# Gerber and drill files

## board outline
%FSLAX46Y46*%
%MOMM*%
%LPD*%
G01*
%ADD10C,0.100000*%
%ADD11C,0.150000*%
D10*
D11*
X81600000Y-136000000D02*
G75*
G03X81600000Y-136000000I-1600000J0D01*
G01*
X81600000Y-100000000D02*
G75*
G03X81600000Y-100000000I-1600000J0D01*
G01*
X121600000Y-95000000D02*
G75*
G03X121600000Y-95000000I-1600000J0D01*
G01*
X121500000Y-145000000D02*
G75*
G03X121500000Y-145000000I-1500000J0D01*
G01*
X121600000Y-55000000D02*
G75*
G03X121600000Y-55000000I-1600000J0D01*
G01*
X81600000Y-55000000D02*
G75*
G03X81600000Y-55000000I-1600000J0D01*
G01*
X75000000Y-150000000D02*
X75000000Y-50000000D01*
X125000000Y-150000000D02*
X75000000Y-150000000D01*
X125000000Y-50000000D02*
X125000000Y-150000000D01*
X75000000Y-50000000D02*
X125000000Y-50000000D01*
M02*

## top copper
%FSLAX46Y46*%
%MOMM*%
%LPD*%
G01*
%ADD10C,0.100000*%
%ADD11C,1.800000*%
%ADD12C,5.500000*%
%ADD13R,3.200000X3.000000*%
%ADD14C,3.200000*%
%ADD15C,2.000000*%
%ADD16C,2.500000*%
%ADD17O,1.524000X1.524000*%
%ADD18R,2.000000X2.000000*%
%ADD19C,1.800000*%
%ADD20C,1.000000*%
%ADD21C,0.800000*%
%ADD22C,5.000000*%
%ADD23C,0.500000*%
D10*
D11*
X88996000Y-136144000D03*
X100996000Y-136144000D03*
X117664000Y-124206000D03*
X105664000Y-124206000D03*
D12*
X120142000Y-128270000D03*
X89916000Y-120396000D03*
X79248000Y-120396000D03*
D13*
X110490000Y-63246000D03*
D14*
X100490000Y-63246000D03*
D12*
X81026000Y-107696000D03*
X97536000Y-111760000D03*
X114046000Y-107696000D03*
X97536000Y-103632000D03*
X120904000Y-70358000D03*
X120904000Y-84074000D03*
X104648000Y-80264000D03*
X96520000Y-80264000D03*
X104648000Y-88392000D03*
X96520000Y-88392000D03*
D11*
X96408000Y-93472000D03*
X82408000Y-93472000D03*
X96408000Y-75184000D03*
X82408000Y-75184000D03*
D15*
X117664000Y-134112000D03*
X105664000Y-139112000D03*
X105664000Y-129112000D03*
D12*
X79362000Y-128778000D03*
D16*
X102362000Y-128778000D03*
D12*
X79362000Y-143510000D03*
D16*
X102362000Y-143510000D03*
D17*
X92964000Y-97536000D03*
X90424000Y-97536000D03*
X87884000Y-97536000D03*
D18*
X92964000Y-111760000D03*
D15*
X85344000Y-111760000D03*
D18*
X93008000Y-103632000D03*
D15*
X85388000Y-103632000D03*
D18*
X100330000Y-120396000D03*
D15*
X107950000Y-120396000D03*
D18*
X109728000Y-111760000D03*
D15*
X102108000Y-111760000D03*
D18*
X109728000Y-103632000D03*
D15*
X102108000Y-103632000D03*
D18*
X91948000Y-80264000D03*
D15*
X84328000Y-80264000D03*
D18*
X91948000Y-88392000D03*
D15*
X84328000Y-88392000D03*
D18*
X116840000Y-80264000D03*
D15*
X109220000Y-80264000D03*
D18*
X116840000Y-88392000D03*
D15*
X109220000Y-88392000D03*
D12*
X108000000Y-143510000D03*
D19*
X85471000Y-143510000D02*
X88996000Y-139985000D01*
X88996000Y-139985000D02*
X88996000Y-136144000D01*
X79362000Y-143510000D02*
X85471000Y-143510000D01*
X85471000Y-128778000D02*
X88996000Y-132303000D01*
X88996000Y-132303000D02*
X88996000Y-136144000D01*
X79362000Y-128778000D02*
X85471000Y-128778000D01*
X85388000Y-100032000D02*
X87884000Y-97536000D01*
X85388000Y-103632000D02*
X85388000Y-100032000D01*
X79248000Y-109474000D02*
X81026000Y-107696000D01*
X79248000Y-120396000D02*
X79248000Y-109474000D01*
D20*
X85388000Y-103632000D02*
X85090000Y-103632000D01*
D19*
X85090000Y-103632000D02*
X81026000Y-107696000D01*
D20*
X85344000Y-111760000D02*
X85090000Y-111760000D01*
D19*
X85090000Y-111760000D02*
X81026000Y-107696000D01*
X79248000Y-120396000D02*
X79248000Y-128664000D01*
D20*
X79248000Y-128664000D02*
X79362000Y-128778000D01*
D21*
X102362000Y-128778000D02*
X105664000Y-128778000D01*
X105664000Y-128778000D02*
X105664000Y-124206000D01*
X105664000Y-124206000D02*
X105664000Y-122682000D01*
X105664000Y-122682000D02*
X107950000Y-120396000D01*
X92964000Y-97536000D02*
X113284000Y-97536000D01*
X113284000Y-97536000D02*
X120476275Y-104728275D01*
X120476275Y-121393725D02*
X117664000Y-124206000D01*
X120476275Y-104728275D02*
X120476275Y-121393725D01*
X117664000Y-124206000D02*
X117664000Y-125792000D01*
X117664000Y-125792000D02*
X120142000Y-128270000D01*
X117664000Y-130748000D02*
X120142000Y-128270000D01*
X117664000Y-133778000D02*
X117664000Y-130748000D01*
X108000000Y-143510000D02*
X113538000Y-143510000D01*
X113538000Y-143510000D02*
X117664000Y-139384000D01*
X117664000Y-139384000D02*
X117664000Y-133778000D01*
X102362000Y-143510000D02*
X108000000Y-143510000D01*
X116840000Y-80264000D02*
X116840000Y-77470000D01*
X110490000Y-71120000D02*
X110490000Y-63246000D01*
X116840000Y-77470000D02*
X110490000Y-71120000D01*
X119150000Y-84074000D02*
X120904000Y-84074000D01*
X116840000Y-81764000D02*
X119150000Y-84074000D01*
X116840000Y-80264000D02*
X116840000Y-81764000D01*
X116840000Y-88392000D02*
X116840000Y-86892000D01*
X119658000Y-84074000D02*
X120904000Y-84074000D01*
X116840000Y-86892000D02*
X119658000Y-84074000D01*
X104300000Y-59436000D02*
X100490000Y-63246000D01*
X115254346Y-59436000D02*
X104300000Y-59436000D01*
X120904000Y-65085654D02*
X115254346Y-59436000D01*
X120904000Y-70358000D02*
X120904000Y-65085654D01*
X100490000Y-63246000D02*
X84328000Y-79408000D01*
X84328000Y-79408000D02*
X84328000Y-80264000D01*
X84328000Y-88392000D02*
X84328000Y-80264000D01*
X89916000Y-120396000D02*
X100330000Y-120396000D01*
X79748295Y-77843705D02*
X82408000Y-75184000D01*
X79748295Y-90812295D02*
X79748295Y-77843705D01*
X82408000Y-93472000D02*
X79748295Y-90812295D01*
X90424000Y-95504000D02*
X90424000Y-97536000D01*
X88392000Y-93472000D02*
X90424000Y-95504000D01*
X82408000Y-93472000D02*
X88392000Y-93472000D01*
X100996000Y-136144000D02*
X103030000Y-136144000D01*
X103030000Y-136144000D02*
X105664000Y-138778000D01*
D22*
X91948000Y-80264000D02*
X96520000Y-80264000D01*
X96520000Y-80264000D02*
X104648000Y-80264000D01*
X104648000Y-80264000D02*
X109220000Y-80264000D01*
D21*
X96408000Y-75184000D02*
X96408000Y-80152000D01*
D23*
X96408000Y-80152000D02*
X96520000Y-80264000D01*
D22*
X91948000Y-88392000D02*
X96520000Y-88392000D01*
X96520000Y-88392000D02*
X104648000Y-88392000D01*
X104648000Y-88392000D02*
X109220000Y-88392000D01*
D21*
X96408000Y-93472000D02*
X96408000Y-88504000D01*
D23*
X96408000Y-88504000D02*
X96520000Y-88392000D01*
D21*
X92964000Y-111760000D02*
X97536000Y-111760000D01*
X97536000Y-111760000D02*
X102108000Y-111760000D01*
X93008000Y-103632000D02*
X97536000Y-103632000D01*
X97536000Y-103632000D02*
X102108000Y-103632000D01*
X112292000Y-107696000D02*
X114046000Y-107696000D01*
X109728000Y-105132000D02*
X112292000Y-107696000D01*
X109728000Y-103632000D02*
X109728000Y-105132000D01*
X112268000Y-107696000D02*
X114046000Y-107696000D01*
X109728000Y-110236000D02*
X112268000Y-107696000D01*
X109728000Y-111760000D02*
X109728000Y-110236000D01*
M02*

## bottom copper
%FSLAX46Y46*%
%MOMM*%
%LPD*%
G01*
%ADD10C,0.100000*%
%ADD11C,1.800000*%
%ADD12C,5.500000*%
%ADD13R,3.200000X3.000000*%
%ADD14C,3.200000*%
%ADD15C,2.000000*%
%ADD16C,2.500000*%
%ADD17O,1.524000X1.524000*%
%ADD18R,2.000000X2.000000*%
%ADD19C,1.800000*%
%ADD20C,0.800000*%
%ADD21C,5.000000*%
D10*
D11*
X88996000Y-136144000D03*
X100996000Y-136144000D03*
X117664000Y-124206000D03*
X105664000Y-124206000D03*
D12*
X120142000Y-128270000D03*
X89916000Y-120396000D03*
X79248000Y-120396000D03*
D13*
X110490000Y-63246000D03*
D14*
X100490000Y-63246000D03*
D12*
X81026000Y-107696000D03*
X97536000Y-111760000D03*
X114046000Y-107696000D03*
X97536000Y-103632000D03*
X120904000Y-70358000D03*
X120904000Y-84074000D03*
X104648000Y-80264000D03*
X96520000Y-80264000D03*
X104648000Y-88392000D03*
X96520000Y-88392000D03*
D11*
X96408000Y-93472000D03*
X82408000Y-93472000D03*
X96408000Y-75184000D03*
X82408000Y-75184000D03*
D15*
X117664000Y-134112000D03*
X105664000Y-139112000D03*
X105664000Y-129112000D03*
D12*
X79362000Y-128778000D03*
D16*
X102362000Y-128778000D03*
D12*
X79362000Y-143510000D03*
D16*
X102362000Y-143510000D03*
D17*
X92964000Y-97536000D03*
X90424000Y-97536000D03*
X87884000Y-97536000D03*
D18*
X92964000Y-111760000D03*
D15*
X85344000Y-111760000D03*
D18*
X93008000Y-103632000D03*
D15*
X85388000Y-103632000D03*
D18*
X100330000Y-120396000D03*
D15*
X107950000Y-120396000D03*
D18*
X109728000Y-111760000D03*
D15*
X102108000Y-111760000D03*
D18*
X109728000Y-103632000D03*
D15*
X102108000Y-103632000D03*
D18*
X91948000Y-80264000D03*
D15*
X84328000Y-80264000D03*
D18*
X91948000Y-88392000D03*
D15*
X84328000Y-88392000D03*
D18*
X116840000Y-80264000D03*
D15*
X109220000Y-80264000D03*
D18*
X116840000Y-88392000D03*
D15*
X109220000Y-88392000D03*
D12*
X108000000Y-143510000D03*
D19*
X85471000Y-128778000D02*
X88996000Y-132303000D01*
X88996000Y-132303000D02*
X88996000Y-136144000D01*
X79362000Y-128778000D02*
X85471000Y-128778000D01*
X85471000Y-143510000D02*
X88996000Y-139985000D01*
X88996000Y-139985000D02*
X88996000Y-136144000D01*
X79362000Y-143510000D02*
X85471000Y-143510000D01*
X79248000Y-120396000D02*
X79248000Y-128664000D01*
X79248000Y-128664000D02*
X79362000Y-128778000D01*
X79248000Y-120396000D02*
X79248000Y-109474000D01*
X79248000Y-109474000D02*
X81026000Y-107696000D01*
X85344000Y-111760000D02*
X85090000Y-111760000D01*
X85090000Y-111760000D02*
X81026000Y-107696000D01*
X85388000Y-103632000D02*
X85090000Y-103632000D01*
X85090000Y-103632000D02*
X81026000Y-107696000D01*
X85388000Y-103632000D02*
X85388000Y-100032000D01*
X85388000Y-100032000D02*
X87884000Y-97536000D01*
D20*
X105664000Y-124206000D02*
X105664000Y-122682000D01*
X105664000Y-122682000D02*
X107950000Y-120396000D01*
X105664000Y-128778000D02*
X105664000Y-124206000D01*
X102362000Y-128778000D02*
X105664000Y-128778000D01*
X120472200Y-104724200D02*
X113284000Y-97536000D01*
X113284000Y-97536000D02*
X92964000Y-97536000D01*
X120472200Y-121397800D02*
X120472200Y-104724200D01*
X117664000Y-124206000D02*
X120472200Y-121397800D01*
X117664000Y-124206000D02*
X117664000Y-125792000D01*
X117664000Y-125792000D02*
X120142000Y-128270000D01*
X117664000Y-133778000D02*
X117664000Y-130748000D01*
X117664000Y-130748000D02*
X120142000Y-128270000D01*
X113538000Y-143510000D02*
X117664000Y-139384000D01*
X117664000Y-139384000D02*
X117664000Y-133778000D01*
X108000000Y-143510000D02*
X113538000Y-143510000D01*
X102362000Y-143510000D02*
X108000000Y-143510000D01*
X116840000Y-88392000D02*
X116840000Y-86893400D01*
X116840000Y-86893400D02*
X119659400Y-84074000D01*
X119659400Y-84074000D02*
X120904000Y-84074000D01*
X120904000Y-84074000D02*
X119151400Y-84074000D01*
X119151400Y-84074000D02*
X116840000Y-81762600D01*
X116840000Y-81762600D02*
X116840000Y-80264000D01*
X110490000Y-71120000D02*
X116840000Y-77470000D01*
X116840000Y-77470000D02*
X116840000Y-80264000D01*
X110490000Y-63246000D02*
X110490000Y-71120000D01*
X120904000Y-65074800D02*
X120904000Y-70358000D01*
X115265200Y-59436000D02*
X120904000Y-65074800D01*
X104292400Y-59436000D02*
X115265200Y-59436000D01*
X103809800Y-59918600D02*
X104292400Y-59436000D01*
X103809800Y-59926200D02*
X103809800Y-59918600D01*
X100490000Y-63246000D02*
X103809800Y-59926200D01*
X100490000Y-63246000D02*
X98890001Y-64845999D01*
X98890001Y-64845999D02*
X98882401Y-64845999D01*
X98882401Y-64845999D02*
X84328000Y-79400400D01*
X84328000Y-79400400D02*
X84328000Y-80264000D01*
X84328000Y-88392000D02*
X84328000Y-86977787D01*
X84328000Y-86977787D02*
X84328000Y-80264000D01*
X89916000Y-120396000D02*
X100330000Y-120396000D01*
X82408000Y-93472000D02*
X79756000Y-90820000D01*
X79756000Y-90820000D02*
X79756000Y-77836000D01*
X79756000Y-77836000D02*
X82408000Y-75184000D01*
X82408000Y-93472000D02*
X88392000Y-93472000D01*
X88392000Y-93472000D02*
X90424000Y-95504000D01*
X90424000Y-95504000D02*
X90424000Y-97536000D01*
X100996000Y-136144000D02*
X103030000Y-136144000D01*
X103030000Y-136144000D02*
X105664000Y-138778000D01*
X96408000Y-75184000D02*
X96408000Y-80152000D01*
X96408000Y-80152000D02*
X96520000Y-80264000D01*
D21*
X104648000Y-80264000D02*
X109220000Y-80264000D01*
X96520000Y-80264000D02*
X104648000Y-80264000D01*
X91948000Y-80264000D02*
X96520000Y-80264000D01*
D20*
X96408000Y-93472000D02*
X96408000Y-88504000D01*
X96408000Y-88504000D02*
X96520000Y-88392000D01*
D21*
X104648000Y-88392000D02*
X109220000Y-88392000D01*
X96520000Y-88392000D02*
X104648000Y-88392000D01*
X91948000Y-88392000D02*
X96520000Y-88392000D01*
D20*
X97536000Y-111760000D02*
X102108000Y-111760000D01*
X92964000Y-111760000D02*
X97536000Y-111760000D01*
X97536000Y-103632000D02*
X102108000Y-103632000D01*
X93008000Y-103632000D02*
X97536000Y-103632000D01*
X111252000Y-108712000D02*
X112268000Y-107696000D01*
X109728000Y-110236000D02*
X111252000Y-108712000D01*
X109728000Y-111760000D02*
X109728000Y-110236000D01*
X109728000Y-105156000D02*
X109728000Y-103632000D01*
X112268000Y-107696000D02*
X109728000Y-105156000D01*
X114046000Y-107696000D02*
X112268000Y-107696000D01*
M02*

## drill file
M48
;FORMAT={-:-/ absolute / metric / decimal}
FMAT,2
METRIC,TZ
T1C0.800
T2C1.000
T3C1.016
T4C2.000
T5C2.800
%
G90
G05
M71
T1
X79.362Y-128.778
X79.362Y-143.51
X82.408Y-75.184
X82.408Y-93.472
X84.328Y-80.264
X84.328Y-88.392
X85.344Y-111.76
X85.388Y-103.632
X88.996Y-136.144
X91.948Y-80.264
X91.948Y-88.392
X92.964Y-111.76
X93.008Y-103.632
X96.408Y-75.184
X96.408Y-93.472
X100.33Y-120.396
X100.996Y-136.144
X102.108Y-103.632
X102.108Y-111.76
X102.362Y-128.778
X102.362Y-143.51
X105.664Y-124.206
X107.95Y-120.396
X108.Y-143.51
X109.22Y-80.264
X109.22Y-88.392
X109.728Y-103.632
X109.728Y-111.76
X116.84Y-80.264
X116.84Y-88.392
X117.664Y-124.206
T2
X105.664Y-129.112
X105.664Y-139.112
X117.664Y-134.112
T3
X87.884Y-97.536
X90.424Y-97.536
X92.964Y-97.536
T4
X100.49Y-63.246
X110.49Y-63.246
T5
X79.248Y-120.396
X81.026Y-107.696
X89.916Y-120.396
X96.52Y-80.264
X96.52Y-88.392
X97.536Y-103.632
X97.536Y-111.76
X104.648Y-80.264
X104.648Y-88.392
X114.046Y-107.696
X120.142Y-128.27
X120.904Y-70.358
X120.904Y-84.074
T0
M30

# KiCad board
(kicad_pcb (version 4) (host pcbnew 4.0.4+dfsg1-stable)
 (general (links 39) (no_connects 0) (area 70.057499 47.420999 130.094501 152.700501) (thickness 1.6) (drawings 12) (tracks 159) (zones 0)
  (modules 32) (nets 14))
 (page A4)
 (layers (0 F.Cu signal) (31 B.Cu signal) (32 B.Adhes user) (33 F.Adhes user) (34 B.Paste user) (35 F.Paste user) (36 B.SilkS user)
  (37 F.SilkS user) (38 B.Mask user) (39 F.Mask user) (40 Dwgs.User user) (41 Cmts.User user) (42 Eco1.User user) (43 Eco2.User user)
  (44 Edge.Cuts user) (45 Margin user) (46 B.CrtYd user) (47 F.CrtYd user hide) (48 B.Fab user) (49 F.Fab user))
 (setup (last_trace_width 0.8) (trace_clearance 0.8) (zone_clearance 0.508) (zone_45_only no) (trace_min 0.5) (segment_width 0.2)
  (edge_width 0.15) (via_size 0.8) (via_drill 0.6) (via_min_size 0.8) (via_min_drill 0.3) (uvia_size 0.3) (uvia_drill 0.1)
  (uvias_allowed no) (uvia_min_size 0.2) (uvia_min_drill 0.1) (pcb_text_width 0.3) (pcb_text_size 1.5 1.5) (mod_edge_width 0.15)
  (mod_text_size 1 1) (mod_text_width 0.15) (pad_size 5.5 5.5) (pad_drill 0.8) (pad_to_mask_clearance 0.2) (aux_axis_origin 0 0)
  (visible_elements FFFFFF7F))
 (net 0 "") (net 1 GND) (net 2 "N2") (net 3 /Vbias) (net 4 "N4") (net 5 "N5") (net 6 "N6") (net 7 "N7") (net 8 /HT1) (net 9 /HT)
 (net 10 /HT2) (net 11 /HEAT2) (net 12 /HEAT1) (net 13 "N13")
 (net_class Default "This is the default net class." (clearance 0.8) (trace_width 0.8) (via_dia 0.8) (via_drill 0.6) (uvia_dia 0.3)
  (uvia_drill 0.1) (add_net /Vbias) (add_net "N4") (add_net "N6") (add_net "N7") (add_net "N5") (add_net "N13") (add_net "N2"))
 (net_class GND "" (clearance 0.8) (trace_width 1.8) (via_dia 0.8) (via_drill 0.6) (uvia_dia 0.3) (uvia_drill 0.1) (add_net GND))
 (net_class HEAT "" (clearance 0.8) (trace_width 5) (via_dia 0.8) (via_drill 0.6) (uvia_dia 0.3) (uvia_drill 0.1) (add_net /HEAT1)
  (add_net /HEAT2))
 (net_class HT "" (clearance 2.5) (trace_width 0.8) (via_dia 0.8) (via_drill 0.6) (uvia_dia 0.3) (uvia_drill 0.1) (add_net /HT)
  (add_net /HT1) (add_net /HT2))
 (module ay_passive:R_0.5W (layer F.Cu) (at 94.996 136.144) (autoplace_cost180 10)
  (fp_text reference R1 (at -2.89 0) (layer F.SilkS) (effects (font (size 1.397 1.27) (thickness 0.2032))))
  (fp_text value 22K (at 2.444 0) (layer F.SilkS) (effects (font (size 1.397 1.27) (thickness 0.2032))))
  (pad 1 thru_hole circle (at -6 0) (size 1.8 1.8) (drill 0.8) (layers *.Cu *.Mask F.SilkS) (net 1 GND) (clearance 0.5))
  (pad 2 thru_hole circle (at 6 0) (size 1.8 1.8) (drill 0.8) (layers *.Cu *.Mask F.SilkS) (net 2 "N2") (clearance 0.5)))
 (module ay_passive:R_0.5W (layer F.Cu) (at 111.664 124.206 180) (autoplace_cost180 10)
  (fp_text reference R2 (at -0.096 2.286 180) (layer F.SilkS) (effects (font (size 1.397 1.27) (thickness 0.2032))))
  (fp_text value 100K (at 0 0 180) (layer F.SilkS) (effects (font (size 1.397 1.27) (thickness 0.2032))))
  (pad 1 thru_hole circle (at -6 0 180) (size 1.8 1.8) (drill 0.8) (layers *.Cu *.Mask F.SilkS) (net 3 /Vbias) (clearance 0.5))
  (pad 2 thru_hole circle (at 6 0 180) (size 1.8 1.8) (drill 0.8) (layers *.Cu *.Mask F.SilkS) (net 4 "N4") (clearance 0.5)))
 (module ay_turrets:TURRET (layer F.Cu) (at 120.142 128.27)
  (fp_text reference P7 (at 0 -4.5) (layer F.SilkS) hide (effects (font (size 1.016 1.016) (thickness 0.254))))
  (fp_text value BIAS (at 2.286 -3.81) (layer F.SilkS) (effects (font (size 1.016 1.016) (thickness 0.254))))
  (pad 1 thru_hole circle (at 0 0) (size 5.5 5.5) (drill 2.8) (layers *.Cu *.Mask F.SilkS) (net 3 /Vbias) (clearance 0.5)))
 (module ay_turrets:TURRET (layer F.Cu) (at 89.916 120.396)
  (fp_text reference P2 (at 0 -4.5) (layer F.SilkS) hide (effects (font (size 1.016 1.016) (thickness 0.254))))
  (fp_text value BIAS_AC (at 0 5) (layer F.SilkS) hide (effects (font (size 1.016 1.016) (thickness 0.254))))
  (pad 1 thru_hole circle (at 0 0) (size 5.5 5.5) (drill 2.8) (layers *.Cu *.Mask F.SilkS) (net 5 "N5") (clearance 0.5)))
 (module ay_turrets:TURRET (layer F.Cu) (at 79.248 120.396)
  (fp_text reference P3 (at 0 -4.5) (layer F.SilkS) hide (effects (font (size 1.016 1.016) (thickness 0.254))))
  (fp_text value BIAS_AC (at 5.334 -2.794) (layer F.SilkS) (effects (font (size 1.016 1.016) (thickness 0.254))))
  (pad 1 thru_hole circle (at 0 0) (size 5.5 5.5) (drill 2.8) (layers *.Cu *.Mask F.SilkS) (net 1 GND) (clearance 0.5)))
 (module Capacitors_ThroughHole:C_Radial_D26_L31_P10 (layer F.Cu) (at 110.49 63.246 180)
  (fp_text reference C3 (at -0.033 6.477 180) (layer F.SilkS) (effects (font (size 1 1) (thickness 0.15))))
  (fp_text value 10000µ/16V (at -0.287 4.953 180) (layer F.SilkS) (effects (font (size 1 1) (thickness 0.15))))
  (pad 1 thru_hole rect (at 0 0 180) (size 3.2 3) (drill 2) (layers *.Cu *.Mask F.SilkS) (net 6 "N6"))
  (pad 2 thru_hole circle (at 10 0 180) (size 3.2 3.2) (drill 2) (layers *.Cu *.Mask F.SilkS) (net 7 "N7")))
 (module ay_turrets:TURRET (layer F.Cu) (at 81.026 107.696)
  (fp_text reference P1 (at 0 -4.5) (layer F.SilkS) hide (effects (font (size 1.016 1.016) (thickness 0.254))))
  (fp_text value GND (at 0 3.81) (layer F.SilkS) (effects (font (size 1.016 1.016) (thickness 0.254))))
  (pad 1 thru_hole circle (at 0 0) (size 5.5 5.5) (drill 2.8) (layers *.Cu *.Mask F.SilkS) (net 1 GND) (clearance 0.5)))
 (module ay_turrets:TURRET (layer F.Cu) (at 97.536 111.76)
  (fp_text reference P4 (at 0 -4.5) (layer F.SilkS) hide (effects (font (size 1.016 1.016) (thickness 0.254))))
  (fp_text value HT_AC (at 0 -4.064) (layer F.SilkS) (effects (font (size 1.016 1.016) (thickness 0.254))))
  (pad 1 thru_hole circle (at 0 0) (size 5.5 5.5) (drill 2.8) (layers *.Cu *.Mask F.SilkS) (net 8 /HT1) (clearance 0.5)))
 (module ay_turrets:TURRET (layer F.Cu) (at 114.046 107.696)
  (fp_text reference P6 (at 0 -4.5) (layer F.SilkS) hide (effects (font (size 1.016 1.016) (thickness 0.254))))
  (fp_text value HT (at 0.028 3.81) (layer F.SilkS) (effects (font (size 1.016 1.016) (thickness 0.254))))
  (pad 1 thru_hole circle (at 0 0) (size 5.5 5.5) (drill 2.8) (layers *.Cu *.Mask F.SilkS) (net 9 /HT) (clearance 0.5)))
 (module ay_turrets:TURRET (layer F.Cu) (at 97.536 103.632)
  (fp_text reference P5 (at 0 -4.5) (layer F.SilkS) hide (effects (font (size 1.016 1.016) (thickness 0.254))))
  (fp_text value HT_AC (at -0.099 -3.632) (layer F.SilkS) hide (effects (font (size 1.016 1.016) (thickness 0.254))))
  (pad 1 thru_hole circle (at 0 0) (size 5.5 5.5) (drill 2.8) (layers *.Cu *.Mask F.SilkS) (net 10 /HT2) (clearance 0.5)))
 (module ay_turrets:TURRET (layer F.Cu) (at 120.904 70.358)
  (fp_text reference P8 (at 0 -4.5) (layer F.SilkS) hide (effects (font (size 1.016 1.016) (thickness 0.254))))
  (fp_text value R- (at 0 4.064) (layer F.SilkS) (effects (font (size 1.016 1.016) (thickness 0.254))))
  (pad 1 thru_hole circle (at 0 0) (size 5.5 5.5) (drill 2.8) (layers *.Cu *.Mask F.SilkS) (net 7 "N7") (clearance 0.5)))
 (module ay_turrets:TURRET (layer F.Cu) (at 120.904 84.074)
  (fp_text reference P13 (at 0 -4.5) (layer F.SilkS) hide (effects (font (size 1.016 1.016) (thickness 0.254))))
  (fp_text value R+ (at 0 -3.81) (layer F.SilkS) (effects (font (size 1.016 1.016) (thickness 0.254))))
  (pad 1 thru_hole circle (at 0 0) (size 5.5 5.5) (drill 2.8) (layers *.Cu *.Mask F.SilkS) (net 6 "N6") (clearance 0.5)))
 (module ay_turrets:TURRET (layer F.Cu) (at 104.648 80.264)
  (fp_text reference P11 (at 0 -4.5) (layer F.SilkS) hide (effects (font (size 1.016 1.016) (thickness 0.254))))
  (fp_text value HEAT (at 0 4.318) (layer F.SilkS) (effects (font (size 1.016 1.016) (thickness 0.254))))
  (pad 1 thru_hole circle (at 0 0) (size 5.5 5.5) (drill 2.8) (layers *.Cu *.Mask F.SilkS) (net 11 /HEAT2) (clearance 0.5)))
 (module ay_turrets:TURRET (layer F.Cu) (at 96.52 80.264)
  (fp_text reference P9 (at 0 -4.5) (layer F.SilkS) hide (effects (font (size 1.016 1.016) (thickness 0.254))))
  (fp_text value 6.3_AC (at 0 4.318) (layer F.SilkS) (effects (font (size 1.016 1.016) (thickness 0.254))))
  (pad 1 thru_hole circle (at 0 0) (size 5.5 5.5) (drill 2.8) (layers *.Cu *.Mask F.SilkS) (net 11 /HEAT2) (clearance 0.5)))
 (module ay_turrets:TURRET (layer F.Cu) (at 104.648 88.392)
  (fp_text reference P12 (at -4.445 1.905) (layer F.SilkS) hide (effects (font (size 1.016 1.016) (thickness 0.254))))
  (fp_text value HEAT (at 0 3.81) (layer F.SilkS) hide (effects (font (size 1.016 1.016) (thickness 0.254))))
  (pad 1 thru_hole circle (at 0 0) (size 5.5 5.5) (drill 2.8) (layers *.Cu *.Mask F.SilkS) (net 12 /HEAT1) (clearance 0.5)))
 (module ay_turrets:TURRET (layer F.Cu) (at 96.52 88.392)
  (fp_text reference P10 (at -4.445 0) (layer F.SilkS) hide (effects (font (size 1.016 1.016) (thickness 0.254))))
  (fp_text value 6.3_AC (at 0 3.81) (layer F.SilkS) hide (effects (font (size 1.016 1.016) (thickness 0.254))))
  (pad 1 thru_hole circle (at 0 0) (size 5.5 5.5) (drill 2.8) (layers *.Cu *.Mask F.SilkS) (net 12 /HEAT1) (clearance 0.5)))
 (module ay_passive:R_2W (layer F.Cu) (at 89.408 93.472 180) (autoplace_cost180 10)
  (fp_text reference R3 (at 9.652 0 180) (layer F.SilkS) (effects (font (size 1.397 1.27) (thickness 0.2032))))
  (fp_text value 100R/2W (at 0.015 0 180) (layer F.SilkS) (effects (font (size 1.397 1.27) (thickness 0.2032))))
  (pad 1 thru_hole circle (at -7 0 180) (size 1.8 1.8) (drill 0.8) (layers *.Cu *.Mask F.SilkS) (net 12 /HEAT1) (clearance 0.5))
  (pad 2 thru_hole circle (at 7 0 180) (size 1.8 1.8) (drill 0.8) (layers *.Cu *.Mask F.SilkS) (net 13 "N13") (clearance 0.5)))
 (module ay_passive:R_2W (layer F.Cu) (at 89.408 75.184 180) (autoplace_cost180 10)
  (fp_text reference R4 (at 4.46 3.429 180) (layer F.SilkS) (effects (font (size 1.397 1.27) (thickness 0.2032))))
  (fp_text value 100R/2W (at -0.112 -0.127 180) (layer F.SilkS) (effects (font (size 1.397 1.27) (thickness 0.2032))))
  (pad 1 thru_hole circle (at -7 0 180) (size 1.8 1.8) (drill 0.8) (layers *.Cu *.Mask F.SilkS) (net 11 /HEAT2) (clearance 0.5))
  (pad 2 thru_hole circle (at 7 0 180) (size 1.8 1.8) (drill 0.8) (layers *.Cu *.Mask F.SilkS) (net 13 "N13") (clearance 0.5)))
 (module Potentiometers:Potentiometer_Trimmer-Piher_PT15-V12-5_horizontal (layer F.Cu) (at 105.664 129.112 270)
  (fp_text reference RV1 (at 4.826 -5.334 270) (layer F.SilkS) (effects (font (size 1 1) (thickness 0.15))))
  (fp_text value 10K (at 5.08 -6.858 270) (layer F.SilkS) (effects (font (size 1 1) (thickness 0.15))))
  (pad 2 thru_hole circle (at 5 -12 270) (size 2 2) (drill 1) (layers *.Cu *.Mask F.SilkS) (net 3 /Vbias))
  (pad 3 thru_hole circle (at 10 0 270) (size 2 2) (drill 1) (layers *.Cu *.Mask F.SilkS) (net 2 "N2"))
  (pad 1 thru_hole circle (at 0 0 270) (size 2 2) (drill 1) (layers *.Cu *.Mask F.SilkS) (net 4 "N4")))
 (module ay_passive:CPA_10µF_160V (layer F.Cu) (at 90.862 128.778 180)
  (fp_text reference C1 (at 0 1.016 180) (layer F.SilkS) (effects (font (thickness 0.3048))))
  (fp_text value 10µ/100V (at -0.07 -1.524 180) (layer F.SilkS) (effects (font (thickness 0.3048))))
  (pad 1 thru_hole circle (at 11.5 0 180) (size 5.5 5.5) (drill 0.8) (layers *.Cu *.Mask F.SilkS) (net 1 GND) (clearance 0.5))
  (pad 2 thru_hole circle (at -11.5 0 180) (size 2.5 2.5) (drill 0.8) (layers *.Cu *.Mask F.SilkS) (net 4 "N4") (clearance 0.5)))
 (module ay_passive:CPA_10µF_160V (layer F.Cu) (at 90.862 143.51 180)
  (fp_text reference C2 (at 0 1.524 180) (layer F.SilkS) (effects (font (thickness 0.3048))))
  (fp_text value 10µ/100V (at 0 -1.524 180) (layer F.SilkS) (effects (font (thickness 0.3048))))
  (pad 1 thru_hole circle (at 11.5 0 180) (size 5.5 5.5) (drill 0.8) (layers *.Cu *.Mask F.SilkS) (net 1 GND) (clearance 0.5))
  (pad 2 thru_hole circle (at -11.5 0 180) (size 2.5 2.5) (drill 0.8) (layers *.Cu *.Mask F.SilkS) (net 3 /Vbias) (clearance 0.5)))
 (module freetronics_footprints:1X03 (layer F.Cu) (at 92.964 97.536 180)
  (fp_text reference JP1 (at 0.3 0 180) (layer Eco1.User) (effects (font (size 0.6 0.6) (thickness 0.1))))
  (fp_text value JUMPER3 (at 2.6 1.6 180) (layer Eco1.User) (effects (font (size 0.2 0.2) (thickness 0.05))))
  (pad 1 thru_hole oval (at 0 0 270) (size 1.524 1.524) (drill 1.016) (layers *.Cu *.Mask) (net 3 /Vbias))
  (pad 2 thru_hole oval (at 2.54 0 270) (size 1.524 1.524) (drill 1.016) (layers *.Cu *.Mask) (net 13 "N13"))
  (pad 3 thru_hole oval (at 5.08 0 270) (size 1.524 1.524) (drill 1.016) (layers *.Cu *.Mask) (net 1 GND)))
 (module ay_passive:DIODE (layer F.Cu) (at 89.154 111.76)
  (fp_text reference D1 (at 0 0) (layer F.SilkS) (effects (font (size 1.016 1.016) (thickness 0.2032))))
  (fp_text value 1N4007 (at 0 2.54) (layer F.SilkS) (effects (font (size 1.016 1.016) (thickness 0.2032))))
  (pad 1 thru_hole rect (at 3.81 0) (size 2 2) (drill 0.8) (layers *.Cu *.Mask F.SilkS) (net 8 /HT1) (clearance 0.5))
  (pad 2 thru_hole circle (at -3.81 0) (size 2 2) (drill 0.8) (layers *.Cu *.Mask F.SilkS) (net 1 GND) (clearance 0.5)))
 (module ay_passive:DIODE (layer F.Cu) (at 89.198 103.632)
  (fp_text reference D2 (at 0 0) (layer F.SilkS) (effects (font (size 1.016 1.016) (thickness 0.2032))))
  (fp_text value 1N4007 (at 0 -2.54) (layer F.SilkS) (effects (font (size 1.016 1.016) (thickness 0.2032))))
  (pad 1 thru_hole rect (at 3.81 0) (size 2 2) (drill 0.8) (layers *.Cu *.Mask F.SilkS) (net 10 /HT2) (clearance 0.5))
  (pad 2 thru_hole circle (at -3.81 0) (size 2 2) (drill 0.8) (layers *.Cu *.Mask F.SilkS) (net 1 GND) (clearance 0.5)))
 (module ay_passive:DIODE (layer F.Cu) (at 104.14 120.396 180)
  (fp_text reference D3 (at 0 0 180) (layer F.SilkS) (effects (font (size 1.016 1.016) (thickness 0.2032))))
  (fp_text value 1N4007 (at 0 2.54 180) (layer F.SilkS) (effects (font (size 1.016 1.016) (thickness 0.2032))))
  (pad 1 thru_hole rect (at 3.81 0 180) (size 2 2) (drill 0.8) (layers *.Cu *.Mask F.SilkS) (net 5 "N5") (clearance 0.5))
  (pad 2 thru_hole circle (at -3.81 0 180) (size 2 2) (drill 0.8) (layers *.Cu *.Mask F.SilkS) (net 4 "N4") (clearance 0.5)))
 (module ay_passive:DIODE (layer F.Cu) (at 105.918 111.76)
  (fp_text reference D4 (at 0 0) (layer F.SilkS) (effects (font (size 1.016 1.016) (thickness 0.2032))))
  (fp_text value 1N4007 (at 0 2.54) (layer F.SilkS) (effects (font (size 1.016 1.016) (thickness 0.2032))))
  (pad 1 thru_hole rect (at 3.81 0) (size 2 2) (drill 0.8) (layers *.Cu *.Mask F.SilkS) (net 9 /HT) (clearance 0.5))
  (pad 2 thru_hole circle (at -3.81 0) (size 2 2) (drill 0.8) (layers *.Cu *.Mask F.SilkS) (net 8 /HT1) (clearance 0.5)))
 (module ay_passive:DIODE (layer F.Cu) (at 105.918 103.632)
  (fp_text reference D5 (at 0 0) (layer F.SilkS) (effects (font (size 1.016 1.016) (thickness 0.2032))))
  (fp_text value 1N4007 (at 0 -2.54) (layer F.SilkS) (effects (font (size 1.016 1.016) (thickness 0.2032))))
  (pad 1 thru_hole rect (at 3.81 0) (size 2 2) (drill 0.8) (layers *.Cu *.Mask F.SilkS) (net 9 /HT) (clearance 0.5))
  (pad 2 thru_hole circle (at -3.81 0) (size 2 2) (drill 0.8) (layers *.Cu *.Mask F.SilkS) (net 10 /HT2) (clearance 0.5)))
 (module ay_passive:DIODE (layer F.Cu) (at 88.138 80.264)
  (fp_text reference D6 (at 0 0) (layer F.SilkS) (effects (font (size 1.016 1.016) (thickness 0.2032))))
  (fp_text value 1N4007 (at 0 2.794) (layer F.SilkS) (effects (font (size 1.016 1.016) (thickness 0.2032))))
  (pad 1 thru_hole rect (at 3.81 0) (size 2 2) (drill 0.8) (layers *.Cu *.Mask F.SilkS) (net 11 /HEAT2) (clearance 0.5))
  (pad 2 thru_hole circle (at -3.81 0) (size 2 2) (drill 0.8) (layers *.Cu *.Mask F.SilkS) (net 7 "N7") (clearance 0.5)))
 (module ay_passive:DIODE (layer F.Cu) (at 88.138 88.392)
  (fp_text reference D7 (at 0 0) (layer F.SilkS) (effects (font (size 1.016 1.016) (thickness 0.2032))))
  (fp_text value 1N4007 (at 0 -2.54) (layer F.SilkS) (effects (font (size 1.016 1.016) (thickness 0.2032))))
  (pad 1 thru_hole rect (at 3.81 0) (size 2 2) (drill 0.8) (layers *.Cu *.Mask F.SilkS) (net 12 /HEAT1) (clearance 0.5))
  (pad 2 thru_hole circle (at -3.81 0) (size 2 2) (drill 0.8) (layers *.Cu *.Mask F.SilkS) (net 7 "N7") (clearance 0.5)))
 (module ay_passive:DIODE (layer F.Cu) (at 113.03 80.264)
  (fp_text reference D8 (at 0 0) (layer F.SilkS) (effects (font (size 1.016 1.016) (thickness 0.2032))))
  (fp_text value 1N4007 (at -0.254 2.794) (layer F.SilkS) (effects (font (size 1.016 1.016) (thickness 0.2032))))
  (pad 1 thru_hole rect (at 3.81 0) (size 2 2) (drill 0.8) (layers *.Cu *.Mask F.SilkS) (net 6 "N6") (clearance 0.5))
  (pad 2 thru_hole circle (at -3.81 0) (size 2 2) (drill 0.8) (layers *.Cu *.Mask F.SilkS) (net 11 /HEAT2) (clearance 0.5)))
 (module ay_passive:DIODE (layer F.Cu) (at 113.03 88.392)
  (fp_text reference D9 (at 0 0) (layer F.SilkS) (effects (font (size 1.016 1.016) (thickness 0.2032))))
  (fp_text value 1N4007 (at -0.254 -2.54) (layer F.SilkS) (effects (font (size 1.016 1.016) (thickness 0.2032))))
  (pad 1 thru_hole rect (at 3.81 0) (size 2 2) (drill 0.8) (layers *.Cu *.Mask F.SilkS) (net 6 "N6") (clearance 0.5))
  (pad 2 thru_hole circle (at -3.81 0) (size 2 2) (drill 0.8) (layers *.Cu *.Mask F.SilkS) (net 12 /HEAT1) (clearance 0.5)))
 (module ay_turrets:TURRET (layer F.Cu) (at 108 143.51)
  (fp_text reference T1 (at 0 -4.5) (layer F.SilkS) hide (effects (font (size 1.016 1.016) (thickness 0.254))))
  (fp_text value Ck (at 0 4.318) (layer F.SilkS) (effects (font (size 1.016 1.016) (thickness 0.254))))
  (pad 1 thru_hole circle (at 0 0) (size 5.5 5.5) (drill 0.8) (layers *.Cu *.Mask F.SilkS) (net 3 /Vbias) (clearance 0.5)))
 (gr_circle (center 80 136) (end 81.6 136) (layer Edge.Cuts) (width 0.15))
 (gr_circle (center 80 100) (end 81.6 100) (layer Edge.Cuts) (width 0.15))
 (gr_circle (center 120 95) (end 121.6 95) (layer Edge.Cuts) (width 0.15))
 (gr_circle (center 120 145) (end 121.5 145) (layer Edge.Cuts) (width 0.15))
 (gr_circle (center 120 55) (end 121.6 55) (layer Edge.Cuts) (width 0.15))
 (gr_circle (center 80 55) (end 81.6 55) (layer Edge.Cuts) (width 0.15))
 (gr_line (start 75 150) (end 75 50) (layer Edge.Cuts) (width 0.15))
 (gr_line (start 125 150) (end 75 150) (layer Edge.Cuts) (width 0.15))
 (gr_line (start 125 50) (end 125 150) (layer Edge.Cuts) (width 0.15))
 (gr_line (start 75 50) (end 125 50) (layer Edge.Cuts) (width 0.15))
 (segment (start 85.471 128.778) (end 88.996 132.303) (width 1.8) (layer B.Cu) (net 1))
 (segment (start 88.996 132.303) (end 88.996 136.144) (width 1.8) (layer B.Cu) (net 1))
 (segment (start 79.362 128.778) (end 85.471 128.778) (width 1.8) (layer B.Cu) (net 1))
 (segment (start 85.471 143.51) (end 88.996 139.985) (width 1.8) (layer B.Cu) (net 1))
 (segment (start 88.996 139.985) (end 88.996 136.144) (width 1.8) (layer B.Cu) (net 1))
 (segment (start 79.362 143.51) (end 85.471 143.51) (width 1.8) (layer B.Cu) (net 1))
 (segment (start 85.471 143.51) (end 88.996 139.985) (width 1.8) (layer F.Cu) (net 1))
 (segment (start 88.996 139.985) (end 88.996 136.144) (width 1.8) (layer F.Cu) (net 1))
 (segment (start 79.362 143.51) (end 85.471 143.51) (width 1.8) (layer F.Cu) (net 1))
 (segment (start 85.471 128.778) (end 88.996 132.303) (width 1.8) (layer F.Cu) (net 1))
 (segment (start 88.996 132.303) (end 88.996 136.144) (width 1.8) (layer F.Cu) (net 1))
 (segment (start 79.362 128.778) (end 85.471 128.778) (width 1.8) (layer F.Cu) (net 1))
 (segment (start 79.248 120.396) (end 79.248 128.664) (width 1.8) (layer B.Cu) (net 1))
 (segment (start 79.248 128.664) (end 79.362 128.778) (width 1.8) (layer B.Cu) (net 1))
 (segment (start 79.248 120.396) (end 79.248 109.474) (width 1.8) (layer B.Cu) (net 1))
 (segment (start 79.248 109.474) (end 81.026 107.696) (width 1.8) (layer B.Cu) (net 1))
 (segment (start 85.344 111.76) (end 85.09 111.76) (width 1.8) (layer B.Cu) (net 1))
 (segment (start 85.09 111.76) (end 81.026 107.696) (width 1.8) (layer B.Cu) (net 1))
 (segment (start 85.388 103.632) (end 85.09 103.632) (width 1.8) (layer B.Cu) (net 1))
 (segment (start 85.09 103.632) (end 81.026 107.696) (width 1.8) (layer B.Cu) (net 1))
 (segment (start 85.388 103.632) (end 85.388 100.032) (width 1.8) (layer B.Cu) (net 1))
 (segment (start 85.388 100.032) (end 87.884 97.536) (width 1.8) (layer B.Cu) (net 1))
 (segment (start 85.388 100.032) (end 87.884 97.536) (width 1.8) (layer F.Cu) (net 1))
 (segment (start 85.388 103.632) (end 85.388 100.032) (width 1.8) (layer F.Cu) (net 1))
 (segment (start 79.248 109.474) (end 81.026 107.696) (width 1.8) (layer F.Cu) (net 1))
 (segment (start 79.248 120.396) (end 79.248 109.474) (width 1.8) (layer F.Cu) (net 1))
 (segment (start 85.388 103.632) (end 85.09 103.632) (width 1) (layer F.Cu) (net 1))
 (segment (start 85.09 103.632) (end 81.026 107.696) (width 1.8) (layer F.Cu) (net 1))
 (segment (start 85.344 111.76) (end 85.09 111.76) (width 1) (layer F.Cu) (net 1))
 (segment (start 85.09 111.76) (end 81.026 107.696) (width 1.8) (layer F.Cu) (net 1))
 (segment (start 79.248 120.396) (end 79.248 128.664) (width 1.8) (layer F.Cu) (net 1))
 (segment (start 79.248 128.664) (end 79.362 128.778) (width 1) (layer F.Cu) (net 1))
 (segment (start 105.664 124.206) (end 105.664 122.682) (width 0.8) (layer B.Cu) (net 4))
 (segment (start 105.664 122.682) (end 107.95 120.396) (width 0.8) (layer B.Cu) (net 4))
 (segment (start 105.664 128.778) (end 105.664 124.206) (width 0.8) (layer B.Cu) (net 4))
 (segment (start 102.362 128.778) (end 105.664 128.778) (width 0.8) (layer B.Cu) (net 4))
 (segment (start 102.362 128.778) (end 105.664 128.778) (width 0.8) (layer F.Cu) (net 4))
 (segment (start 105.664 128.778) (end 105.664 124.206) (width 0.8) (layer F.Cu) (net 4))
 (segment (start 105.664 124.206) (end 105.664 122.682) (width 0.8) (layer F.Cu) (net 4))
 (segment (start 105.664 122.682) (end 107.95 120.396) (width 0.8) (layer F.Cu) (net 4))
 (segment (start 120.4722 104.7242) (end 113.284 97.536) (width 0.8) (layer B.Cu) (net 3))
 (segment (start 113.284 97.536) (end 92.964 97.536) (width 0.8) (layer B.Cu) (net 3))
 (segment (start 120.4722 121.3978) (end 120.4722 104.7242) (width 0.8) (layer B.Cu) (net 3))
 (segment (start 117.664 124.206) (end 120.4722 121.3978) (width 0.8) (layer B.Cu) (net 3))
 (segment (start 117.664 124.206) (end 117.664 125.792) (width 0.8) (layer B.Cu) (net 3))
 (segment (start 117.664 125.792) (end 120.142 128.27) (width 0.8) (layer B.Cu) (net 3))
 (segment (start 117.664 133.778) (end 117.664 130.748) (width 0.8) (layer B.Cu) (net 3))
 (segment (start 117.664 130.748) (end 120.142 128.27) (width 0.8) (layer B.Cu) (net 3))
 (segment (start 113.538 143.51) (end 117.664 139.384) (width 0.8) (layer B.Cu) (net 3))
 (segment (start 117.664 139.384) (end 117.664 133.778) (width 0.8) (layer B.Cu) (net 3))
 (segment (start 108 143.51) (end 113.538 143.51) (width 0.8) (layer B.Cu) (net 3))
 (segment (start 102.362 143.51) (end 108 143.51) (width 0.8) (layer B.Cu) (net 3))
 (segment (start 92.964 97.536) (end 113.284 97.536) (width 0.8) (layer F.Cu) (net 3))
 (segment (start 113.284 97.536) (end 120.476275 104.728275) (width 0.8) (layer F.Cu) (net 3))
 (segment (start 120.476275 121.393725) (end 117.664 124.206) (width 0.8) (layer F.Cu) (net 3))
 (segment (start 120.476275 104.728275) (end 120.476275 121.393725) (width 0.8) (layer F.Cu) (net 3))
 (segment (start 117.664 124.206) (end 117.664 125.792) (width 0.8) (layer F.Cu) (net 3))
 (segment (start 117.664 125.792) (end 120.142 128.27) (width 0.8) (layer F.Cu) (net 3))
 (segment (start 117.664 130.748) (end 120.142 128.27) (width 0.8) (layer F.Cu) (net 3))
 (segment (start 117.664 133.778) (end 117.664 130.748) (width 0.8) (layer F.Cu) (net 3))
 (segment (start 108 143.51) (end 113.538 143.51) (width 0.8) (layer F.Cu) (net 3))
 (segment (start 113.538 143.51) (end 117.664 139.384) (width 0.8) (layer F.Cu) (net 3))
 (segment (start 117.664 139.384) (end 117.664 133.778) (width 0.8) (layer F.Cu) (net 3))
 (segment (start 102.362 143.51) (end 108 143.51) (width 0.8) (layer F.Cu) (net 3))
 (segment (start 116.84 88.392) (end 116.84 86.8934) (width 0.8) (layer B.Cu) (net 6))
 (segment (start 116.84 86.8934) (end 119.6594 84.074) (width 0.8) (layer B.Cu) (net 6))
 (segment (start 119.6594 84.074) (end 120.904 84.074) (width 0.8) (layer B.Cu) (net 6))
 (segment (start 120.904 84.074) (end 119.1514 84.074) (width 0.8) (layer B.Cu) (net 6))
 (segment (start 119.1514 84.074) (end 116.84 81.7626) (width 0.8) (layer B.Cu) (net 6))
 (segment (start 116.84 81.7626) (end 116.84 80.264) (width 0.8) (layer B.Cu) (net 6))
 (segment (start 110.49 71.12) (end 116.84 77.47) (width 0.8) (layer B.Cu) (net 6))
 (segment (start 116.84 77.47) (end 116.84 80.264) (width 0.8) (layer B.Cu) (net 6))
 (segment (start 110.49 63.246) (end 110.49 71.12) (width 0.8) (layer B.Cu) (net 6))
 (segment (start 116.84 80.264) (end 116.84 77.47) (width 0.8) (layer F.Cu) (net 6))
 (segment (start 110.49 71.12) (end 110.49 63.246) (width 0.8) (layer F.Cu) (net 6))
 (segment (start 116.84 77.47) (end 110.49 71.12) (width 0.8) (layer F.Cu) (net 6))
 (segment (start 119.15 84.074) (end 120.904 84.074) (width 0.8) (layer F.Cu) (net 6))
 (segment (start 116.84 81.764) (end 119.15 84.074) (width 0.8) (layer F.Cu) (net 6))
 (segment (start 116.84 80.264) (end 116.84 81.764) (width 0.8) (layer F.Cu) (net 6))
 (segment (start 116.84 88.392) (end 116.84 86.892) (width 0.8) (layer F.Cu) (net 6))
 (segment (start 119.658 84.074) (end 120.904 84.074) (width 0.8) (layer F.Cu) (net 6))
 (segment (start 116.84 86.892) (end 119.658 84.074) (width 0.8) (layer F.Cu) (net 6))
 (segment (start 120.904 65.0748) (end 120.904 70.358) (width 0.8) (layer B.Cu) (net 7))
 (segment (start 115.2652 59.436) (end 120.904 65.0748) (width 0.8) (layer B.Cu) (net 7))
 (segment (start 104.2924 59.436) (end 115.2652 59.436) (width 0.8) (layer B.Cu) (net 7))
 (segment (start 103.8098 59.9186) (end 104.2924 59.436) (width 0.8) (layer B.Cu) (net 7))
 (segment (start 103.8098 59.9262) (end 103.8098 59.9186) (width 0.8) (layer B.Cu) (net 7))
 (segment (start 100.49 63.246) (end 103.8098 59.9262) (width 0.8) (layer B.Cu) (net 7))
 (segment (start 100.49 63.246) (end 98.890001 64.845999) (width 0.8) (layer B.Cu) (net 7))
 (segment (start 98.890001 64.845999) (end 98.882401 64.845999) (width 0.8) (layer B.Cu) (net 7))
 (segment (start 98.882401 64.845999) (end 84.328 79.4004) (width 0.8) (layer B.Cu) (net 7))
 (segment (start 84.328 79.4004) (end 84.328 80.264) (width 0.8) (layer B.Cu) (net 7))
 (segment (start 84.328 88.392) (end 84.328 86.977787) (width 0.8) (layer B.Cu) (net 7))
 (segment (start 84.328 86.977787) (end 84.328 80.264) (width 0.8) (layer B.Cu) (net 7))
 (segment (start 104.3 59.436) (end 100.49 63.246) (width 0.8) (layer F.Cu) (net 7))
 (segment (start 115.254346 59.436) (end 104.3 59.436) (width 0.8) (layer F.Cu) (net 7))
 (segment (start 120.904 65.085654) (end 115.254346 59.436) (width 0.8) (layer F.Cu) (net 7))
 (segment (start 120.904 70.358) (end 120.904 65.085654) (width 0.8) (layer F.Cu) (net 7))
 (segment (start 100.49 63.246) (end 84.328 79.408) (width 0.8) (layer F.Cu) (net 7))
 (segment (start 84.328 79.408) (end 84.328 80.264) (width 0.8) (layer F.Cu) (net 7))
 (segment (start 84.328 88.392) (end 84.328 80.264) (width 0.8) (layer F.Cu) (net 7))
 (segment (start 89.916 120.396) (end 100.33 120.396) (width 0.8) (layer B.Cu) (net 5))
 (segment (start 89.916 120.396) (end 100.33 120.396) (width 0.8) (layer F.Cu) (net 5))
 (segment (start 82.408 93.472) (end 79.756 90.82) (width 0.8) (layer B.Cu) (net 13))
 (segment (start 79.756 90.82) (end 79.756 77.836) (width 0.8) (layer B.Cu) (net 13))
 (segment (start 79.756 77.836) (end 82.408 75.184) (width 0.8) (layer B.Cu) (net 13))
 (segment (start 82.408 93.472) (end 88.392 93.472) (width 0.8) (layer B.Cu) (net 13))
 (segment (start 88.392 93.472) (end 90.424 95.504) (width 0.8) (layer B.Cu) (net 13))
 (segment (start 90.424 95.504) (end 90.424 97.536) (width 0.8) (layer B.Cu) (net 13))
 (segment (start 79.748295 77.843705) (end 82.408 75.184) (width 0.8) (layer F.Cu) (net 13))
 (segment (start 79.748295 90.812295) (end 79.748295 77.843705) (width 0.8) (layer F.Cu) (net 13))
 (segment (start 82.408 93.472) (end 79.748295 90.812295) (width 0.8) (layer F.Cu) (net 13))
 (segment (start 90.424 95.504) (end 90.424 97.536) (width 0.8) (layer F.Cu) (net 13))
 (segment (start 88.392 93.472) (end 90.424 95.504) (width 0.8) (layer F.Cu) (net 13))
 (segment (start 82.408 93.472) (end 88.392 93.472) (width 0.8) (layer F.Cu) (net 13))
 (segment (start 100.996 136.144) (end 103.03 136.144) (width 0.8) (layer B.Cu) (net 2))
 (segment (start 103.03 136.144) (end 105.664 138.778) (width 0.8) (layer B.Cu) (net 2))
 (segment (start 100.996 136.144) (end 103.03 136.144) (width 0.8) (layer F.Cu) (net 2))
 (segment (start 103.03 136.144) (end 105.664 138.778) (width 0.8) (layer F.Cu) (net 2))
 (segment (start 96.408 75.184) (end 96.408 80.152) (width 0.8) (layer B.Cu) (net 11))
 (segment (start 96.408 80.152) (end 96.52 80.264) (width 0.8) (layer B.Cu) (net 11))
 (segment (start 104.648 80.264) (end 109.22 80.264) (width 5) (layer B.Cu) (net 11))
 (segment (start 96.52 80.264) (end 104.648 80.264) (width 5) (layer B.Cu) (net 11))
 (segment (start 91.948 80.264) (end 96.52 80.264) (width 5) (layer B.Cu) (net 11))
 (segment (start 91.948 80.264) (end 96.52 80.264) (width 5) (layer F.Cu) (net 11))
 (segment (start 96.52 80.264) (end 104.648 80.264) (width 5) (layer F.Cu) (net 11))
 (segment (start 104.648 80.264) (end 109.22 80.264) (width 5) (layer F.Cu) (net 11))
 (segment (start 96.408 75.184) (end 96.408 80.152) (width 0.8) (layer F.Cu) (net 11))
 (segment (start 96.408 80.152) (end 96.52 80.264) (width 0.5) (layer F.Cu) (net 11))
 (segment (start 96.408 93.472) (end 96.408 88.504) (width 0.8) (layer B.Cu) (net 12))
 (segment (start 96.408 88.504) (end 96.52 88.392) (width 0.8) (layer B.Cu) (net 12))
 (segment (start 104.648 88.392) (end 109.22 88.392) (width 5) (layer B.Cu) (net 12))
 (segment (start 96.52 88.392) (end 104.648 88.392) (width 5) (layer B.Cu) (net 12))
 (segment (start 91.948 88.392) (end 96.52 88.392) (width 5) (layer B.Cu) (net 12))
 (segment (start 91.948 88.392) (end 96.52 88.392) (width 5) (layer F.Cu) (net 12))
 (segment (start 96.52 88.392) (end 104.648 88.392) (width 5) (layer F.Cu) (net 12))
 (segment (start 104.648 88.392) (end 109.22 88.392) (width 5) (layer F.Cu) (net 12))
 (segment (start 96.408 93.472) (end 96.408 88.504) (width 0.8) (layer F.Cu) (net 12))
 (segment (start 96.408 88.504) (end 96.52 88.392) (width 0.5) (layer F.Cu) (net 12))
 (segment (start 97.536 111.76) (end 102.108 111.76) (width 0.8) (layer B.Cu) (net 8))
 (segment (start 92.964 111.76) (end 97.536 111.76) (width 0.8) (layer B.Cu) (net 8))
 (segment (start 92.964 111.76) (end 97.536 111.76) (width 0.8) (layer F.Cu) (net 8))
 (segment (start 97.536 111.76) (end 102.108 111.76) (width 0.8) (layer F.Cu) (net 8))
 (segment (start 97.536 103.632) (end 102.108 103.632) (width 0.8) (layer B.Cu) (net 10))
 (segment (start 93.008 103.632) (end 97.536 103.632) (width 0.8) (layer B.Cu) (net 10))
 (segment (start 93.008 103.632) (end 97.536 103.632) (width 0.8) (layer F.Cu) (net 10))
 (segment (start 97.536 103.632) (end 102.108 103.632) (width 0.8) (layer F.Cu) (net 10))
 (segment (start 111.252 108.712) (end 112.268 107.696) (width 0.8) (layer B.Cu) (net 9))
 (segment (start 109.728 110.236) (end 111.252 108.712) (width 0.8) (layer B.Cu) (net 9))
 (segment (start 109.728 111.76) (end 109.728 110.236) (width 0.8) (layer B.Cu) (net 9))
 (segment (start 109.728 105.156) (end 109.728 103.632) (width 0.8) (layer B.Cu) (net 9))
 (segment (start 112.268 107.696) (end 109.728 105.156) (width 0.8) (layer B.Cu) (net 9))
 (segment (start 114.046 107.696) (end 112.268 107.696) (width 0.8) (layer B.Cu) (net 9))
 (segment (start 112.292 107.696) (end 114.046 107.696) (width 0.8) (layer F.Cu) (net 9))
 (segment (start 109.728 105.132) (end 112.292 107.696) (width 0.8) (layer F.Cu) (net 9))
 (segment (start 109.728 103.632) (end 109.728 105.132) (width 0.8) (layer F.Cu) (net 9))
 (segment (start 112.268 107.696) (end 114.046 107.696) (width 0.8) (layer F.Cu) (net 9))
 (segment (start 109.728 110.236) (end 112.268 107.696) (width 0.8) (layer F.Cu) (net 9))
 (segment (start 109.728 111.76) (end 109.728 110.236) (width 0.8) (layer F.Cu) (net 9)))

